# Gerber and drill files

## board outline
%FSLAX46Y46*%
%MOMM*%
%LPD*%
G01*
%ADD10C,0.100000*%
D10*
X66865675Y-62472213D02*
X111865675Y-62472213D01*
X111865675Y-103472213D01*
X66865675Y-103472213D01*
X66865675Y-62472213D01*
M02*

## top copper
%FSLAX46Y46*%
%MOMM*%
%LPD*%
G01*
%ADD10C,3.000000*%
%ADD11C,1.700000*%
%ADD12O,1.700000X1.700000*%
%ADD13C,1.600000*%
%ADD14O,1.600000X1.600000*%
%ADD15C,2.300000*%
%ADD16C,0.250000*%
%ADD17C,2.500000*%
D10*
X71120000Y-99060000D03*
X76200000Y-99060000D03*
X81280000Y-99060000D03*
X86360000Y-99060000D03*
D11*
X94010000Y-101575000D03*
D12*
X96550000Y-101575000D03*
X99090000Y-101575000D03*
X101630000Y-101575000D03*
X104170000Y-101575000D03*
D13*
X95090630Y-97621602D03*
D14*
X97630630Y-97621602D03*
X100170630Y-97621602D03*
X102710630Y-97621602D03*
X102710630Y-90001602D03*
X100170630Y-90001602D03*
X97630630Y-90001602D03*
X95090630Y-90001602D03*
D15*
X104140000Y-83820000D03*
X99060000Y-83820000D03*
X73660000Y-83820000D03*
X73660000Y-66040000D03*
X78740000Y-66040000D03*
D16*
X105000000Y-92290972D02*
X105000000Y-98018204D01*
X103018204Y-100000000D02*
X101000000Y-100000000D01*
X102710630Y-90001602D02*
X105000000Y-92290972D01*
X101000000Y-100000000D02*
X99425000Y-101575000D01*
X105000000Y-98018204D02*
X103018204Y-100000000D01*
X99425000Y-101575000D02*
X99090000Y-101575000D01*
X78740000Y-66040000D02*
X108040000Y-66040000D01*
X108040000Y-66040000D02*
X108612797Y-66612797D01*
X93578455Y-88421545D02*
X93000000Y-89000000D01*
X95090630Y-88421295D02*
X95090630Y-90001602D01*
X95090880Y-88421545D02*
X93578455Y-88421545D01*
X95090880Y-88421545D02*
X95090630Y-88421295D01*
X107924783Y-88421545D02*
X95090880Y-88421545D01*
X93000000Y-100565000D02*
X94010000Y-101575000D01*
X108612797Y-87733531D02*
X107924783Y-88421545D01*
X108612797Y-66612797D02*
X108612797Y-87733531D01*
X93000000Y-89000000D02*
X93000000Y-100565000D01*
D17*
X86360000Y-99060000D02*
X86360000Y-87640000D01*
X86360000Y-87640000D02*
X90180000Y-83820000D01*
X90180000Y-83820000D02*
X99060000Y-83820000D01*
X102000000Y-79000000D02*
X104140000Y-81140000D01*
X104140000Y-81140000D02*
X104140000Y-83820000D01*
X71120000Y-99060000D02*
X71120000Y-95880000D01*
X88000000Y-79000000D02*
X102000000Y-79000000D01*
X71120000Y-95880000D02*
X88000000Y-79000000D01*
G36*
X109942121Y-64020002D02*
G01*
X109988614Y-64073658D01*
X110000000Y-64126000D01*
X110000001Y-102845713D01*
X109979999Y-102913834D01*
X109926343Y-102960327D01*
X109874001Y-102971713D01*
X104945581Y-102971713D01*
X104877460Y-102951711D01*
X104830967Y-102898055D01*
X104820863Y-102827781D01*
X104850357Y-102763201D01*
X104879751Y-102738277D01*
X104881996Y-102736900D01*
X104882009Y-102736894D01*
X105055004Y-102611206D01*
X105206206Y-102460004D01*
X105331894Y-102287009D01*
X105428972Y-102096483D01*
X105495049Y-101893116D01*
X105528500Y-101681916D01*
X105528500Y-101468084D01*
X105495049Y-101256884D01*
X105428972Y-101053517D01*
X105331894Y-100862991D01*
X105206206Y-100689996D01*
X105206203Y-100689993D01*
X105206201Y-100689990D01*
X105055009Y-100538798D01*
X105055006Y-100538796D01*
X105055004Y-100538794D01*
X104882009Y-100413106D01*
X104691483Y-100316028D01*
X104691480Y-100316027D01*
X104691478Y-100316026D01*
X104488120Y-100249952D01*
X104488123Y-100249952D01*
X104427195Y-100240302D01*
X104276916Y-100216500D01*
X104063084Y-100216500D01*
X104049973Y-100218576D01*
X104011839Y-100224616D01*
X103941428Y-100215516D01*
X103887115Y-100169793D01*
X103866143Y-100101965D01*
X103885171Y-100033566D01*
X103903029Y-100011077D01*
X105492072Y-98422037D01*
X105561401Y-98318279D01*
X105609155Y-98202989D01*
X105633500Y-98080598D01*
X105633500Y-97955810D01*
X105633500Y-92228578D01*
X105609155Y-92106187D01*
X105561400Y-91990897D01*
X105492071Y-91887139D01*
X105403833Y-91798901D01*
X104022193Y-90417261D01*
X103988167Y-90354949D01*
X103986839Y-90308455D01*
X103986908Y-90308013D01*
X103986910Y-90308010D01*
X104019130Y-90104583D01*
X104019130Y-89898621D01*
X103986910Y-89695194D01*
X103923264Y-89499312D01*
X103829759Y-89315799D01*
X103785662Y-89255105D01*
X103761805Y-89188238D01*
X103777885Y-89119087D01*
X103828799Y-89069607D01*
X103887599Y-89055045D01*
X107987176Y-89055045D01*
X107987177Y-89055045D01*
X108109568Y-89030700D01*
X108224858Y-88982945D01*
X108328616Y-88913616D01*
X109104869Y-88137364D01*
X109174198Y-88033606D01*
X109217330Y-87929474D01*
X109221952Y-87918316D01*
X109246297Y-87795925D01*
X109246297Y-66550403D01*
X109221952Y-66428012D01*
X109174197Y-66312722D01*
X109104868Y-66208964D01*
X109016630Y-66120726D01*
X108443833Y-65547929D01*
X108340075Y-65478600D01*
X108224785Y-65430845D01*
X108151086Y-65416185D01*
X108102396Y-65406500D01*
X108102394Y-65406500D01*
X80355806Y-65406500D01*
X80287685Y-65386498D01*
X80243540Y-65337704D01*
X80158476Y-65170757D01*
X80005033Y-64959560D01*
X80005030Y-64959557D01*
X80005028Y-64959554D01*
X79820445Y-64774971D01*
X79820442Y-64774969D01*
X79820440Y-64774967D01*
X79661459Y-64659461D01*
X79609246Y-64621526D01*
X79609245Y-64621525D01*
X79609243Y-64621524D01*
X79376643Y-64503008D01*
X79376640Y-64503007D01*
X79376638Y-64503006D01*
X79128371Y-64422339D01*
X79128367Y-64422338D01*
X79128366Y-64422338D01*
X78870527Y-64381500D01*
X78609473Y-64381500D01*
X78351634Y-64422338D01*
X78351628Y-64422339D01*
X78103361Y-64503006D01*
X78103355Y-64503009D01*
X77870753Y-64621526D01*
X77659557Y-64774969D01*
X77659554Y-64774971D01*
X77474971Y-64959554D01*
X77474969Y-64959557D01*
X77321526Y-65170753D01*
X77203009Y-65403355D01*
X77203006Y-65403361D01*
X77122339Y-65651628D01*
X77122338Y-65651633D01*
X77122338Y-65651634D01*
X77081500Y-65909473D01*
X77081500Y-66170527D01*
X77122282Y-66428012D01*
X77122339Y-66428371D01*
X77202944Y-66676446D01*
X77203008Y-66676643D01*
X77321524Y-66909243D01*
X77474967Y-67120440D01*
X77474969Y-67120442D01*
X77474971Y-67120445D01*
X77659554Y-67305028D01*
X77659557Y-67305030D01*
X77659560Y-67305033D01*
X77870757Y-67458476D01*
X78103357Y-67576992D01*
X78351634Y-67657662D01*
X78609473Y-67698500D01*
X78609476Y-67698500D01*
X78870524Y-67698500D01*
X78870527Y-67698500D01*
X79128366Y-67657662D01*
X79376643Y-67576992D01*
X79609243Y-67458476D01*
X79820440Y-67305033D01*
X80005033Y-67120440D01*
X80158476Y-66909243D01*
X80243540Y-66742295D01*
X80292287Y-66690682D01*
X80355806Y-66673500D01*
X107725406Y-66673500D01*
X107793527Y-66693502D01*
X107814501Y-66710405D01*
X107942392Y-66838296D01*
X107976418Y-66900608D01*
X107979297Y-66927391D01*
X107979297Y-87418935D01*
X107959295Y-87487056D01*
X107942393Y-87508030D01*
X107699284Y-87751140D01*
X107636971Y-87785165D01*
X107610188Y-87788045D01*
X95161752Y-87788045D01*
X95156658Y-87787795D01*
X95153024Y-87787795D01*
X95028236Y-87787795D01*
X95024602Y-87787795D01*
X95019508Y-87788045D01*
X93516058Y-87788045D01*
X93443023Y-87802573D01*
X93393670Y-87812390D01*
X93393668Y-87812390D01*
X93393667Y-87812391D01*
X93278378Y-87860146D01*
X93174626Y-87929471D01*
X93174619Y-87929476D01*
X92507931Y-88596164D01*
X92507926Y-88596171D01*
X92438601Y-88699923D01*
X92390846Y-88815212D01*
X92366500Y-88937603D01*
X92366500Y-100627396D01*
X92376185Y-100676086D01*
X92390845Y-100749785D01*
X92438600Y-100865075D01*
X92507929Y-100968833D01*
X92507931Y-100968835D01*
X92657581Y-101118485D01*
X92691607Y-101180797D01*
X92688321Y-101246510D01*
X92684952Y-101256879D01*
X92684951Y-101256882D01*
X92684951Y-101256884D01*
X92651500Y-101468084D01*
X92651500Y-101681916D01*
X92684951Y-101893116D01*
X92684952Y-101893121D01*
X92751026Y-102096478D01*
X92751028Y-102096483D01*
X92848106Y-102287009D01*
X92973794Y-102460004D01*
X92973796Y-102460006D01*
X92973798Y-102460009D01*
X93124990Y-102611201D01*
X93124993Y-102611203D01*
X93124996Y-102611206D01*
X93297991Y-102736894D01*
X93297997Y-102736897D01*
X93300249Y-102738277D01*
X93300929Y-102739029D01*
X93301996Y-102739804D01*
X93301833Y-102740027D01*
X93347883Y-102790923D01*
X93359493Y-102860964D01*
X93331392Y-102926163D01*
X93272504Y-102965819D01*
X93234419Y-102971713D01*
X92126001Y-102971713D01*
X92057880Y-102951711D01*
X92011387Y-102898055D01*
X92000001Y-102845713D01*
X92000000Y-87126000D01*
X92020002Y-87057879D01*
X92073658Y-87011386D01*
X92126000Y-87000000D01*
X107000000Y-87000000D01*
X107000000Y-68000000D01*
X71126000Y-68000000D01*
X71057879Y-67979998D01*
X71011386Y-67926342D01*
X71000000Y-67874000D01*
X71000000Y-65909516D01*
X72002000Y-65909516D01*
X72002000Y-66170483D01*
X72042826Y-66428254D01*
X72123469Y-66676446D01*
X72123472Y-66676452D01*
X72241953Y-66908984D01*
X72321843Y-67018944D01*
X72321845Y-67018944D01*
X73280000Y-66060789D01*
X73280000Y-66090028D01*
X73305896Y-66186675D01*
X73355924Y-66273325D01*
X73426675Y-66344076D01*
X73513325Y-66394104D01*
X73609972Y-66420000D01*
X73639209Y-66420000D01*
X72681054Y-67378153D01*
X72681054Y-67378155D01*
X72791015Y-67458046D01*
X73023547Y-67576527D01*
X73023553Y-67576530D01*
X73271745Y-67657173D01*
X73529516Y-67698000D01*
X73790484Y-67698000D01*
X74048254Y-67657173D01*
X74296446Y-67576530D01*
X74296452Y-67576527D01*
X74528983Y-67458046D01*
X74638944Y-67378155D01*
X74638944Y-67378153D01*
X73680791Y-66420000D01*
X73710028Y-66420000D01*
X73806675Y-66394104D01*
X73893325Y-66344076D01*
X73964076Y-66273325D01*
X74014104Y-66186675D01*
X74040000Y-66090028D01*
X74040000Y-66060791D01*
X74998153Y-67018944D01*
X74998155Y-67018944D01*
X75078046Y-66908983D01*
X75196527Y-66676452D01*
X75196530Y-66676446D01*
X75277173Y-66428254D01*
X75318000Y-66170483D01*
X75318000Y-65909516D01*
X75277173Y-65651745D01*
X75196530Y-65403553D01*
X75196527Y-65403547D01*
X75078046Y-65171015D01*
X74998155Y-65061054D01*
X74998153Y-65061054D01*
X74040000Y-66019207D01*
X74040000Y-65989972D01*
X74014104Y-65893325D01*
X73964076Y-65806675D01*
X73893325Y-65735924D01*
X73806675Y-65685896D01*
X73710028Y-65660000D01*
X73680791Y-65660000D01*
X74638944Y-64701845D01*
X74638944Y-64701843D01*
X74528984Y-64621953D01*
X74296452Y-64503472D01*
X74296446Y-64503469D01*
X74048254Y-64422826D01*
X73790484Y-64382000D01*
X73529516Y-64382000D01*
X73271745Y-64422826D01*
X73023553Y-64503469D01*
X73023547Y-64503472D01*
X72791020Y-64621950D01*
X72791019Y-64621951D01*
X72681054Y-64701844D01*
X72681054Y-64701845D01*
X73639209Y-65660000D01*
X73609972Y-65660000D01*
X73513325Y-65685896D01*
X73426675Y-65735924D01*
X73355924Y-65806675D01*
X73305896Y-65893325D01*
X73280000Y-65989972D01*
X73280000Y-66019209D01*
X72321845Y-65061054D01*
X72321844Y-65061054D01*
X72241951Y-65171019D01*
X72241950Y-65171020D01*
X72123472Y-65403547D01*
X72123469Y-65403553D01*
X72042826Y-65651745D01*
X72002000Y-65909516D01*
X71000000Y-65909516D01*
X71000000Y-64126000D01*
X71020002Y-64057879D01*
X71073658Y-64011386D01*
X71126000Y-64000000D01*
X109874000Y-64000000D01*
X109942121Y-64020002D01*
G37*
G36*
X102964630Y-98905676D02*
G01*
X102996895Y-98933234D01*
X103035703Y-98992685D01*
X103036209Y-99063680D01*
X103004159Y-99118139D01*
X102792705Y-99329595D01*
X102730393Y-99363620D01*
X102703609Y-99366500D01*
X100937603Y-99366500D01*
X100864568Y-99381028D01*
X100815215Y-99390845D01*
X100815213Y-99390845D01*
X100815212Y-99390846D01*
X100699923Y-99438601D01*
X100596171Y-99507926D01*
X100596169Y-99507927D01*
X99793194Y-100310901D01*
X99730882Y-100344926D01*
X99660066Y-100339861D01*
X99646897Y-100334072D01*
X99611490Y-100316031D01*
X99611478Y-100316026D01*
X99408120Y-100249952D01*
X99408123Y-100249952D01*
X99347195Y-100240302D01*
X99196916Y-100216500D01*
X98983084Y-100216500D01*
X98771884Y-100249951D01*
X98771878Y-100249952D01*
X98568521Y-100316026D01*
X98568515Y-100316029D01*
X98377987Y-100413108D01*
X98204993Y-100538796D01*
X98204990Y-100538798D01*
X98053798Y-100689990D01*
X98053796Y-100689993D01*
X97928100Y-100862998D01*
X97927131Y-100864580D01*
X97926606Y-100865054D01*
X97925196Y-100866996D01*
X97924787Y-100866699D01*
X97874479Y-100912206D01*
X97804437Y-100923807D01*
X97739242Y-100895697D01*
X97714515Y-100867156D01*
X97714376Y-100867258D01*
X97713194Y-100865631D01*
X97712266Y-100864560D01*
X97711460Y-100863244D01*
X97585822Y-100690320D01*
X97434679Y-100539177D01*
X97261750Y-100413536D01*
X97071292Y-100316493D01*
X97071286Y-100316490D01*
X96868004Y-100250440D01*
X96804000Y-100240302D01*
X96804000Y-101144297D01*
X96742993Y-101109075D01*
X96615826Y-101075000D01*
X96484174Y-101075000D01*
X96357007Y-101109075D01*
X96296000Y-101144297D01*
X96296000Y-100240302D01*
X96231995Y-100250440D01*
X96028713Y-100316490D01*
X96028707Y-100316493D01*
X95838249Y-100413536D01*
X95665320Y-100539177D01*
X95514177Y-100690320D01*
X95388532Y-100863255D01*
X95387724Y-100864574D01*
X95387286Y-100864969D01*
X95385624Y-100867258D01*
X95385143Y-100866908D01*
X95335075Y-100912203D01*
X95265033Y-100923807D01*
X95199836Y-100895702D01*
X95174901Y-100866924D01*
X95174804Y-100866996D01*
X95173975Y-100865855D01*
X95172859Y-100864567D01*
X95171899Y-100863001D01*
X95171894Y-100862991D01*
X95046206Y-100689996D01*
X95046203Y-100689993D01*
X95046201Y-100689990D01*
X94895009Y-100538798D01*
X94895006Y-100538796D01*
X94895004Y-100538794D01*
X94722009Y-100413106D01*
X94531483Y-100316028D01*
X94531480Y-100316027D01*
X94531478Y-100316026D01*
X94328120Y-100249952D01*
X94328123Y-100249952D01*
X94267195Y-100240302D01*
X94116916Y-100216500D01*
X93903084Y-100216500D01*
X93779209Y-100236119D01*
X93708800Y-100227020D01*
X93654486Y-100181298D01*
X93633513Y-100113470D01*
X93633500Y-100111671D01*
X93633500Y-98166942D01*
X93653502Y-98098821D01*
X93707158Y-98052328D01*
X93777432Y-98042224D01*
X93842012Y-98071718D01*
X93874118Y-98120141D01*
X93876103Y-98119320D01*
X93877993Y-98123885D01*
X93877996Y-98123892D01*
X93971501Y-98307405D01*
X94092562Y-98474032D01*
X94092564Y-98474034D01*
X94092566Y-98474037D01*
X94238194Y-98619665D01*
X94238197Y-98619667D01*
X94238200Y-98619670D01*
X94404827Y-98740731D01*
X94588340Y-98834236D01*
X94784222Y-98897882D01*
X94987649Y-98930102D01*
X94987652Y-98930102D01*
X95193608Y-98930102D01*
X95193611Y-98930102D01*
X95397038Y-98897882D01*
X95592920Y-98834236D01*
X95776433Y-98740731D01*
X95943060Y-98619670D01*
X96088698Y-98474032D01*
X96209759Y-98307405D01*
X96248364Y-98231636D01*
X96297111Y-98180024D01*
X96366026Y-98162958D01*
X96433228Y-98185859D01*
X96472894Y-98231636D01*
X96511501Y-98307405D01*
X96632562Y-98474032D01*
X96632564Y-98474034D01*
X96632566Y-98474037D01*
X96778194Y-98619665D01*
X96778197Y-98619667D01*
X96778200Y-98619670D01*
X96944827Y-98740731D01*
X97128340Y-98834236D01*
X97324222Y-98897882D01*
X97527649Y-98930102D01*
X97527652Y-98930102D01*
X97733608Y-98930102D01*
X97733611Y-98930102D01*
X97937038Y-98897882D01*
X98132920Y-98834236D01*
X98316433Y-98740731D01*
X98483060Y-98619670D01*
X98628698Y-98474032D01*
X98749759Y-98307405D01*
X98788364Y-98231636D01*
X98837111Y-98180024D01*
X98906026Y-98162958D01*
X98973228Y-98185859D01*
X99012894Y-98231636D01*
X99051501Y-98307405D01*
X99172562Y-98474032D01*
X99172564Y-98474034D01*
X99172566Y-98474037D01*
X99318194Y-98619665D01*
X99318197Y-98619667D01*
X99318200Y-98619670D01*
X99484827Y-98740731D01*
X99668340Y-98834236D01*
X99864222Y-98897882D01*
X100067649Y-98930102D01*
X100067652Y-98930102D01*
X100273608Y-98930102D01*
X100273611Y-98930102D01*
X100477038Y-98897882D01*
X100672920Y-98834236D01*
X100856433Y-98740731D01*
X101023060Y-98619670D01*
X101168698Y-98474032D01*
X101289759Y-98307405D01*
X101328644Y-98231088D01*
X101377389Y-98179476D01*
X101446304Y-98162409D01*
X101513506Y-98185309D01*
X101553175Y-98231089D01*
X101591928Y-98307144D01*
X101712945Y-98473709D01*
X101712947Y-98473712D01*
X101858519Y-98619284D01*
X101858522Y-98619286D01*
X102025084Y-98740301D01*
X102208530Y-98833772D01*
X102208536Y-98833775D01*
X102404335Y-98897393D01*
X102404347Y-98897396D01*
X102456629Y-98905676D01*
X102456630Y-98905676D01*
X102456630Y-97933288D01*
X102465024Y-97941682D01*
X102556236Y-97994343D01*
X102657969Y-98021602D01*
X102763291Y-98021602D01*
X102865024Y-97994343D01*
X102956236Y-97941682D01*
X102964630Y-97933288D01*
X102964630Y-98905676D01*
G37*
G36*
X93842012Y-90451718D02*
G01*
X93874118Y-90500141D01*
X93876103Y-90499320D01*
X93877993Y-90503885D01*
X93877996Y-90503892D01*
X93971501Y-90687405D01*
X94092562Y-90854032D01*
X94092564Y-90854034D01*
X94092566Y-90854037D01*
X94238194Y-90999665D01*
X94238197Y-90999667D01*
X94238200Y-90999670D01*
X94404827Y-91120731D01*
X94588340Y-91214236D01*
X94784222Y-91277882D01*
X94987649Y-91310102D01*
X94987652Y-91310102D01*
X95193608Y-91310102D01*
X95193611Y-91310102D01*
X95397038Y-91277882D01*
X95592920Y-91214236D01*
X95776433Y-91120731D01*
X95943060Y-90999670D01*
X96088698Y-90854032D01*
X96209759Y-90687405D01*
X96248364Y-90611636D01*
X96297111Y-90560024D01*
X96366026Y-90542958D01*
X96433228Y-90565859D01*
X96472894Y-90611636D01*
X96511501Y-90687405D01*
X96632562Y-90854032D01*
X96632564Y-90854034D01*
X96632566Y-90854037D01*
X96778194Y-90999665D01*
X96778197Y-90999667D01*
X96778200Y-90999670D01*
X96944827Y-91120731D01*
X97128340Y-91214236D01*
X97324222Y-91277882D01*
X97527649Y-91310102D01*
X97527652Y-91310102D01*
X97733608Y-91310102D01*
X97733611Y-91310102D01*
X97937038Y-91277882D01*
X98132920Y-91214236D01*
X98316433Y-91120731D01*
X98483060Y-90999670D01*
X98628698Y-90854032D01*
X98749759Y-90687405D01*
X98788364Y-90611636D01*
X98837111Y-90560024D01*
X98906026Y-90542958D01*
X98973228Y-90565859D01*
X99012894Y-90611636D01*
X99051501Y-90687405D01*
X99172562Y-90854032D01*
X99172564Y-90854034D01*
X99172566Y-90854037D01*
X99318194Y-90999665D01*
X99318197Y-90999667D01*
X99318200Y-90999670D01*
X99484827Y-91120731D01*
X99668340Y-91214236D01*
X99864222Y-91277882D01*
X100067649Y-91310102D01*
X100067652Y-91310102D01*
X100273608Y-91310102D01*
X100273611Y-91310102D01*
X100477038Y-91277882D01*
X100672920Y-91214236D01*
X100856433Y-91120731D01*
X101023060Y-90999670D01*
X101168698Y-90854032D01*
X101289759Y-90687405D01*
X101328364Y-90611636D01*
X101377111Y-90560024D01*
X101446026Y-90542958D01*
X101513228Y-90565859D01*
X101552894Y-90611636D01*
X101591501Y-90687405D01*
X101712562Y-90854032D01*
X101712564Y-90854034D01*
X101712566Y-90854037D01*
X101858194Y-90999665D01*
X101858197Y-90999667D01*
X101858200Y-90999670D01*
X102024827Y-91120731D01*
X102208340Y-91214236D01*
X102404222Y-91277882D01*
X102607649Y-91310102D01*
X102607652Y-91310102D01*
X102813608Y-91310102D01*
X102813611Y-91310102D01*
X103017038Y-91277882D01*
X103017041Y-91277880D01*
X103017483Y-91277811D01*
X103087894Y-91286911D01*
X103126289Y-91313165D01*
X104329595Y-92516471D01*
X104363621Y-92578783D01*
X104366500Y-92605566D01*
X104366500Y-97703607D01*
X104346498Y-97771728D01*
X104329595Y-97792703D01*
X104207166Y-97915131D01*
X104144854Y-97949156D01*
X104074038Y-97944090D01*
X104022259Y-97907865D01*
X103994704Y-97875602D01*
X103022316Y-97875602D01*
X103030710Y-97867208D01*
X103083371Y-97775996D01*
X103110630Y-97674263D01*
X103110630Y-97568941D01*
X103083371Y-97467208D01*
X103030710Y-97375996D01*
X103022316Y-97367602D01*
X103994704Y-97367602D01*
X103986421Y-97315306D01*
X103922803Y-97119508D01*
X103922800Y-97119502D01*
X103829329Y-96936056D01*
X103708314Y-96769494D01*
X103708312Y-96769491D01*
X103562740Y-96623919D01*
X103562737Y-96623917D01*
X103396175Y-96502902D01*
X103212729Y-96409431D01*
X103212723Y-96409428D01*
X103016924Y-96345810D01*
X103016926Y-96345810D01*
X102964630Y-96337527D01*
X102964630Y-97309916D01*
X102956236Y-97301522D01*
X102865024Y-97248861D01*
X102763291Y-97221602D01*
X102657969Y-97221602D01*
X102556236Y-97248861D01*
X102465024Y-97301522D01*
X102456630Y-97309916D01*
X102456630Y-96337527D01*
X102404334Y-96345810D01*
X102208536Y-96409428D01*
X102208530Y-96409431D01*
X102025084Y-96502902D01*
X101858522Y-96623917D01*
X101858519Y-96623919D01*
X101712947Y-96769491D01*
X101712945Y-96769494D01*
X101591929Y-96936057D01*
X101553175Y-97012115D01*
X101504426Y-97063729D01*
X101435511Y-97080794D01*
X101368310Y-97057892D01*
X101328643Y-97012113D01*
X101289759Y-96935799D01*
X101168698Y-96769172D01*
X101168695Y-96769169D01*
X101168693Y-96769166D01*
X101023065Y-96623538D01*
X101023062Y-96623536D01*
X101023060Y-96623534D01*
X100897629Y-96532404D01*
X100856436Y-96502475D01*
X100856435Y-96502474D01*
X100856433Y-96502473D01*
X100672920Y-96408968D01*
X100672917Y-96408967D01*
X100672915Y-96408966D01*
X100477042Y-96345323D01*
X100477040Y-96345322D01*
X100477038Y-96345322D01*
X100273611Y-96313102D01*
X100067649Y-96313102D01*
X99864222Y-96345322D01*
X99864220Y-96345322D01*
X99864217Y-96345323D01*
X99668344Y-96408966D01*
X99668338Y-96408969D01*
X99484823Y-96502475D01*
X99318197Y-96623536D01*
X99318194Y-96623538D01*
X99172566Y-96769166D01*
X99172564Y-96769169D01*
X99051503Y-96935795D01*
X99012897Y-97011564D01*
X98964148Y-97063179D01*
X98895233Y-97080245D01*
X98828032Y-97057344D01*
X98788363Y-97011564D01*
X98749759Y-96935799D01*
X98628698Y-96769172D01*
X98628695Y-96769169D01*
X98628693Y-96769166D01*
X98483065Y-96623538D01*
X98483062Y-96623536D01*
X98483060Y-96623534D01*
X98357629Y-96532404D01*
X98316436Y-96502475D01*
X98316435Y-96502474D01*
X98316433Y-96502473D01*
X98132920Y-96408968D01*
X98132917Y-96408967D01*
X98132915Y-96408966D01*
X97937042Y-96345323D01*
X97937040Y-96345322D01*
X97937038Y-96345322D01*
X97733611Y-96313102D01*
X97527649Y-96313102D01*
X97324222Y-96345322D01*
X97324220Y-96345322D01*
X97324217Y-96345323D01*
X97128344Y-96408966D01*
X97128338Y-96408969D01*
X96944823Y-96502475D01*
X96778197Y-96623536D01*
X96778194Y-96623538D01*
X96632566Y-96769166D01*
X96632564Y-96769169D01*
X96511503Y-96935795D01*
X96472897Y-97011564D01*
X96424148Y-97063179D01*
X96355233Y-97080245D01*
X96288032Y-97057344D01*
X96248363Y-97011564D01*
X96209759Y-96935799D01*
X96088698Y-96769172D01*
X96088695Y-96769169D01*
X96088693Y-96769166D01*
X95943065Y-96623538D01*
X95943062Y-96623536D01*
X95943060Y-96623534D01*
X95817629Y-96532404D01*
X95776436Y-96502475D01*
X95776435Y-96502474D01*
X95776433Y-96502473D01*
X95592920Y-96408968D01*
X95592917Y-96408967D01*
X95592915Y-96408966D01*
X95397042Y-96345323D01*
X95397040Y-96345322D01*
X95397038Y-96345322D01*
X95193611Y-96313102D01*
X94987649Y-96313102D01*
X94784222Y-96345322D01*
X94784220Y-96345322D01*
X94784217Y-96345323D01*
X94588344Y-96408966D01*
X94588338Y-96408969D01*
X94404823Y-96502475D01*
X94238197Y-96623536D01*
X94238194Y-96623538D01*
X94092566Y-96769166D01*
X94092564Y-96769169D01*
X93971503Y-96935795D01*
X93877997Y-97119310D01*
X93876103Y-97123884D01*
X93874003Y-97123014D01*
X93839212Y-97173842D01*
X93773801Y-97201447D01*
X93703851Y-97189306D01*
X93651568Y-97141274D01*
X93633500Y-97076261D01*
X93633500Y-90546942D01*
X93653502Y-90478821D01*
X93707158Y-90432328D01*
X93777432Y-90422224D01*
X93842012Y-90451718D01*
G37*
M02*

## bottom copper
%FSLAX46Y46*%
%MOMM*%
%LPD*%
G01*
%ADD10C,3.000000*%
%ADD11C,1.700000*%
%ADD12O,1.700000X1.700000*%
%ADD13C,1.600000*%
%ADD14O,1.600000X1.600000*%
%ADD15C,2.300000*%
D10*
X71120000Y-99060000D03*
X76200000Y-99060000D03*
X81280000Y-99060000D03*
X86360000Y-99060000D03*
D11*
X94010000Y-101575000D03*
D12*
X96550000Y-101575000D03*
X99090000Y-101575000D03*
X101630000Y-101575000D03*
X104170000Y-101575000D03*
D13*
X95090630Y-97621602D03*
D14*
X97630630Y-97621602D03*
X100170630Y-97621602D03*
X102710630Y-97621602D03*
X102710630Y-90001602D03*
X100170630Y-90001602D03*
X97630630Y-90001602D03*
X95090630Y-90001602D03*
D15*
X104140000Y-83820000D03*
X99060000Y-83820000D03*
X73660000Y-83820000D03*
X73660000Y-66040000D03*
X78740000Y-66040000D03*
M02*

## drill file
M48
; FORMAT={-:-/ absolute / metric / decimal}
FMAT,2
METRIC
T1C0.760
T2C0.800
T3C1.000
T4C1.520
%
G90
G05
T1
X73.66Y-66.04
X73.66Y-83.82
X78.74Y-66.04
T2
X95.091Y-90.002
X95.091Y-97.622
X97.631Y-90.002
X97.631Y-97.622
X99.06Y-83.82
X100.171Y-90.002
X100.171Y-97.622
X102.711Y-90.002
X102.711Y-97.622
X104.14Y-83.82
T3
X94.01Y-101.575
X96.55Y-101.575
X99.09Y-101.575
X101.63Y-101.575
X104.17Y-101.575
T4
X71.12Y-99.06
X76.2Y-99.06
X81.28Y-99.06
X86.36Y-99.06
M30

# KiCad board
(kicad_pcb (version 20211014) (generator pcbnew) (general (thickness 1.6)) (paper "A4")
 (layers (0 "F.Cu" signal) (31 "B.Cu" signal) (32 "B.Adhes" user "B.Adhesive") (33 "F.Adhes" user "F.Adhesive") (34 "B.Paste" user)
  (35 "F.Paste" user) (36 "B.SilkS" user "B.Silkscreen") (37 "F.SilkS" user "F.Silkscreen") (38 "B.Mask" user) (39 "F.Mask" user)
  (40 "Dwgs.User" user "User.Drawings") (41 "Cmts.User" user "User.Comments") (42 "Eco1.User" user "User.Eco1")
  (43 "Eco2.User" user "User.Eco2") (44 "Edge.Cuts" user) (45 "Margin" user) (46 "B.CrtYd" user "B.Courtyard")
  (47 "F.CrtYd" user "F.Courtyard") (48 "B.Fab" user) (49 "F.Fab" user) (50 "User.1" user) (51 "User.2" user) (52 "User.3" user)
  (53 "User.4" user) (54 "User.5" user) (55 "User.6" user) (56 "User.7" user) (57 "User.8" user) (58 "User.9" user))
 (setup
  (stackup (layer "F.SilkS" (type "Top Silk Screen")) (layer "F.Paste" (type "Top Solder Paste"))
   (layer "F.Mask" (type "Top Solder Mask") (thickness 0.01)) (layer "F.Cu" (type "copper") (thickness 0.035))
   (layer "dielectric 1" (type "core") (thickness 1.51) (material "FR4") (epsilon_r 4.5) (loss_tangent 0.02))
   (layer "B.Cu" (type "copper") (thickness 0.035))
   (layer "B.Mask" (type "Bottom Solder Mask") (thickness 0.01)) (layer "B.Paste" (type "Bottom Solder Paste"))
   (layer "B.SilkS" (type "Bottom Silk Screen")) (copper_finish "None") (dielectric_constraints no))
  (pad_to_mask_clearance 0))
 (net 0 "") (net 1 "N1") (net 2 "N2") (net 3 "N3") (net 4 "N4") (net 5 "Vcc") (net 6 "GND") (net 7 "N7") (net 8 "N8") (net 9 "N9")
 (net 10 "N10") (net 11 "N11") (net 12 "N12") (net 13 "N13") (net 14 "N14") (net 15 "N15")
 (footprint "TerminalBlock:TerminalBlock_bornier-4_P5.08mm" (layer "F.Cu") (at 71.12 99.06)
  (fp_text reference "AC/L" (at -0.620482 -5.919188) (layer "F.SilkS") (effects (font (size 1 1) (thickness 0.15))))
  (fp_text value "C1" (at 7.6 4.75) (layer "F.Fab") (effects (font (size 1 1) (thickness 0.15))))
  (pad "1" thru_hole circle (at 0 0) (size 3 3) (drill 1.52) (layers *.Cu *.Mask) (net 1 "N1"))
  (pad "2" thru_hole circle (at 5.08 0) (size 3 3) (drill 1.52) (layers *.Cu *.Mask) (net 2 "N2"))
  (pad "3" thru_hole circle (at 10.16 0) (size 3 3) (drill 1.52) (layers *.Cu *.Mask) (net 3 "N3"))
  (pad "4" thru_hole circle (at 15.24 0) (size 3 3) (drill 1.52) (layers *.Cu *.Mask) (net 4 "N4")))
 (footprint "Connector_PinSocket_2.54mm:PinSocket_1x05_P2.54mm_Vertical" (layer "F.Cu") (at 94.01 101.575 90)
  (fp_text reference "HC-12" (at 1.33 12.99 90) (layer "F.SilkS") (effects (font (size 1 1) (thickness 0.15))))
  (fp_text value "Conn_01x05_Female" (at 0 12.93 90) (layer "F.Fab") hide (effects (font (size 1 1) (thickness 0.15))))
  (pad "1" thru_hole circle (at 0 0 90) (size 1.7 1.7) (drill 1) (layers *.Cu *.Mask) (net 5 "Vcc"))
  (pad "2" thru_hole oval (at 0 2.54 90) (size 1.7 1.7) (drill 1) (layers *.Cu *.Mask) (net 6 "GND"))
  (pad "3" thru_hole oval (at 0 5.08 90) (size 1.7 1.7) (drill 1) (layers *.Cu *.Mask) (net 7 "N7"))
  (pad "4" thru_hole oval (at 0 7.62 90) (size 1.7 1.7) (drill 1) (layers *.Cu *.Mask) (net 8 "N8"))
  (pad "5" thru_hole oval (at 0 10.16 90) (size 1.7 1.7) (drill 1) (layers *.Cu *.Mask) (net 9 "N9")))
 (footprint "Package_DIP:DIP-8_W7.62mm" (layer "F.Cu") (at 95.09063 97.621602 90)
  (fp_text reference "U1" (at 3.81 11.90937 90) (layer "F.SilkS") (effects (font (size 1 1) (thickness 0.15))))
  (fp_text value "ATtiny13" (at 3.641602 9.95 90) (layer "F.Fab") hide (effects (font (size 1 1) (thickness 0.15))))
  (pad "1" thru_hole circle (at 0 0 90) (size 1.6 1.6) (drill 0.8) (layers *.Cu *.Mask) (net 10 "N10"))
  (pad "2" thru_hole oval (at 0 2.54 90) (size 1.6 1.6) (drill 0.8) (layers *.Cu *.Mask) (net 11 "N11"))
  (pad "3" thru_hole oval (at 0 5.08 90) (size 1.6 1.6) (drill 0.8) (layers *.Cu *.Mask) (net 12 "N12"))
  (pad "4" thru_hole oval (at 0 7.62 90) (size 1.6 1.6) (drill 0.8) (layers *.Cu *.Mask) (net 6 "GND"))
  (pad "5" thru_hole oval (at 7.62 7.62 90) (size 1.6 1.6) (drill 0.8) (layers *.Cu *.Mask) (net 7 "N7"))
  (pad "6" thru_hole oval (at 7.62 5.08 90) (size 1.6 1.6) (drill 0.8) (layers *.Cu *.Mask) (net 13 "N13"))
  (pad "7" thru_hole oval (at 7.62 2.54 90) (size 1.6 1.6) (drill 0.8) (layers *.Cu *.Mask) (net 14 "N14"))
  (pad "8" thru_hole oval (at 7.62 0 90) (size 1.6 1.6) (drill 0.8) (layers *.Cu *.Mask) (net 5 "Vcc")))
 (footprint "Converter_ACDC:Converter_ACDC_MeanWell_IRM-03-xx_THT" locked (layer "B.Cu") (at 104.14 83.82 90)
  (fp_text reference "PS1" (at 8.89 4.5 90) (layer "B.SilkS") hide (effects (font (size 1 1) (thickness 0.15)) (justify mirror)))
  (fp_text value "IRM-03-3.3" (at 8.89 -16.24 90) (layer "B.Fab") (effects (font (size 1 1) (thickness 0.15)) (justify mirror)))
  (pad "1" thru_hole circle locked (at 0 0 90) (size 2.3 2.3) (drill 0.8) (layers *.Cu *.Mask) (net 1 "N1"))
  (pad "3" thru_hole circle locked (at 0 -5.08 90) (size 2.3 2.3) (drill 0.8) (layers *.Cu *.Mask) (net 4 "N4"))
  (pad "5" thru_hole circle locked (at 0 -30.48 90) (size 2.3 2.3) (drill 0.76) (layers *.Cu *.Mask) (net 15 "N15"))
  (pad "14" thru_hole circle locked (at 17.78 -30.48 90) (size 2.3 2.3) (drill 0.76) (layers *.Cu *.Mask) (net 6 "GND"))
  (pad "16" thru_hole circle locked (at 17.78 -25.4 90) (size 2.3 2.3) (drill 0.76) (layers *.Cu *.Mask) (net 5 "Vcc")))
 (gr_rect (start 66.865675 62.472213) (end 111.865675 103.472213) (layer "Edge.Cuts") (width 0.1) (fill none))
 (segment (start 105 92.290972) (end 105 98.018204) (width 0.25) (layer "F.Cu") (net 7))
 (segment (start 103.018204 100) (end 101 100) (width 0.25) (layer "F.Cu") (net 7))
 (segment (start 102.71063 90.001602) (end 105 92.290972) (width 0.25) (layer "F.Cu") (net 7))
 (segment (start 101 100) (end 99.425 101.575) (width 0.25) (layer "F.Cu") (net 7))
 (segment (start 105 98.018204) (end 103.018204 100) (width 0.25) (layer "F.Cu") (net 7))
 (segment (start 99.425 101.575) (end 99.09 101.575) (width 0.25) (layer "F.Cu") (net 7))
 (segment (start 78.74 66.04) (end 108.04 66.04) (width 0.25) (layer "F.Cu") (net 5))
 (segment (start 108.04 66.04) (end 108.612797 66.612797) (width 0.25) (layer "F.Cu") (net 5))
 (segment (start 93.578455 88.421545) (end 93 89) (width 0.25) (layer "F.Cu") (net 5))
 (segment (start 95.09063 88.421295) (end 95.09063 90.001602) (width 0.25) (layer "F.Cu") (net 5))
 (segment (start 95.09088 88.421545) (end 93.578455 88.421545) (width 0.25) (layer "F.Cu") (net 5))
 (segment (start 95.09088 88.421545) (end 95.09063 88.421295) (width 0.25) (layer "F.Cu") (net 5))
 (segment (start 107.924783 88.421545) (end 95.09088 88.421545) (width 0.25) (layer "F.Cu") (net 5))
 (segment (start 93 100.565) (end 94.01 101.575) (width 0.25) (layer "F.Cu") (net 5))
 (segment (start 108.612797 87.733531) (end 107.924783 88.421545) (width 0.25) (layer "F.Cu") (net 5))
 (segment (start 108.612797 66.612797) (end 108.612797 87.733531) (width 0.25) (layer "F.Cu") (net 5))
 (segment (start 93 89) (end 93 100.565) (width 0.25) (layer "F.Cu") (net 5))
 (segment (start 86.36 99.06) (end 86.36 87.64) (width 2.5) (layer "F.Cu") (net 4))
 (segment (start 86.36 87.64) (end 90.18 83.82) (width 2.5) (layer "F.Cu") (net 4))
 (segment (start 90.18 83.82) (end 99.06 83.82) (width 2.5) (layer "F.Cu") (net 4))
 (segment (start 102 79) (end 104.14 81.14) (width 2.5) (layer "F.Cu") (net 1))
 (segment (start 104.14 81.14) (end 104.14 83.82) (width 2.5) (layer "F.Cu") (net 1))
 (segment (start 71.12 99.06) (end 71.12 95.88) (width 2.5) (layer "F.Cu") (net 1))
 (segment (start 88 79) (end 102 79) (width 2.5) (layer "F.Cu") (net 1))
 (segment (start 71.12 95.88) (end 88 79) (width 2.5) (layer "F.Cu") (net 1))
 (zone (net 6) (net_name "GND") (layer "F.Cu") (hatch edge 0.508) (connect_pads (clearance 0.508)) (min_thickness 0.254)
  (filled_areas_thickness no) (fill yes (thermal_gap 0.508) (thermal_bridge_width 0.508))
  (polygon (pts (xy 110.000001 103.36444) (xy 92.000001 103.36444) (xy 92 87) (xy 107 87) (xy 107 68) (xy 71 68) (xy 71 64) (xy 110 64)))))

